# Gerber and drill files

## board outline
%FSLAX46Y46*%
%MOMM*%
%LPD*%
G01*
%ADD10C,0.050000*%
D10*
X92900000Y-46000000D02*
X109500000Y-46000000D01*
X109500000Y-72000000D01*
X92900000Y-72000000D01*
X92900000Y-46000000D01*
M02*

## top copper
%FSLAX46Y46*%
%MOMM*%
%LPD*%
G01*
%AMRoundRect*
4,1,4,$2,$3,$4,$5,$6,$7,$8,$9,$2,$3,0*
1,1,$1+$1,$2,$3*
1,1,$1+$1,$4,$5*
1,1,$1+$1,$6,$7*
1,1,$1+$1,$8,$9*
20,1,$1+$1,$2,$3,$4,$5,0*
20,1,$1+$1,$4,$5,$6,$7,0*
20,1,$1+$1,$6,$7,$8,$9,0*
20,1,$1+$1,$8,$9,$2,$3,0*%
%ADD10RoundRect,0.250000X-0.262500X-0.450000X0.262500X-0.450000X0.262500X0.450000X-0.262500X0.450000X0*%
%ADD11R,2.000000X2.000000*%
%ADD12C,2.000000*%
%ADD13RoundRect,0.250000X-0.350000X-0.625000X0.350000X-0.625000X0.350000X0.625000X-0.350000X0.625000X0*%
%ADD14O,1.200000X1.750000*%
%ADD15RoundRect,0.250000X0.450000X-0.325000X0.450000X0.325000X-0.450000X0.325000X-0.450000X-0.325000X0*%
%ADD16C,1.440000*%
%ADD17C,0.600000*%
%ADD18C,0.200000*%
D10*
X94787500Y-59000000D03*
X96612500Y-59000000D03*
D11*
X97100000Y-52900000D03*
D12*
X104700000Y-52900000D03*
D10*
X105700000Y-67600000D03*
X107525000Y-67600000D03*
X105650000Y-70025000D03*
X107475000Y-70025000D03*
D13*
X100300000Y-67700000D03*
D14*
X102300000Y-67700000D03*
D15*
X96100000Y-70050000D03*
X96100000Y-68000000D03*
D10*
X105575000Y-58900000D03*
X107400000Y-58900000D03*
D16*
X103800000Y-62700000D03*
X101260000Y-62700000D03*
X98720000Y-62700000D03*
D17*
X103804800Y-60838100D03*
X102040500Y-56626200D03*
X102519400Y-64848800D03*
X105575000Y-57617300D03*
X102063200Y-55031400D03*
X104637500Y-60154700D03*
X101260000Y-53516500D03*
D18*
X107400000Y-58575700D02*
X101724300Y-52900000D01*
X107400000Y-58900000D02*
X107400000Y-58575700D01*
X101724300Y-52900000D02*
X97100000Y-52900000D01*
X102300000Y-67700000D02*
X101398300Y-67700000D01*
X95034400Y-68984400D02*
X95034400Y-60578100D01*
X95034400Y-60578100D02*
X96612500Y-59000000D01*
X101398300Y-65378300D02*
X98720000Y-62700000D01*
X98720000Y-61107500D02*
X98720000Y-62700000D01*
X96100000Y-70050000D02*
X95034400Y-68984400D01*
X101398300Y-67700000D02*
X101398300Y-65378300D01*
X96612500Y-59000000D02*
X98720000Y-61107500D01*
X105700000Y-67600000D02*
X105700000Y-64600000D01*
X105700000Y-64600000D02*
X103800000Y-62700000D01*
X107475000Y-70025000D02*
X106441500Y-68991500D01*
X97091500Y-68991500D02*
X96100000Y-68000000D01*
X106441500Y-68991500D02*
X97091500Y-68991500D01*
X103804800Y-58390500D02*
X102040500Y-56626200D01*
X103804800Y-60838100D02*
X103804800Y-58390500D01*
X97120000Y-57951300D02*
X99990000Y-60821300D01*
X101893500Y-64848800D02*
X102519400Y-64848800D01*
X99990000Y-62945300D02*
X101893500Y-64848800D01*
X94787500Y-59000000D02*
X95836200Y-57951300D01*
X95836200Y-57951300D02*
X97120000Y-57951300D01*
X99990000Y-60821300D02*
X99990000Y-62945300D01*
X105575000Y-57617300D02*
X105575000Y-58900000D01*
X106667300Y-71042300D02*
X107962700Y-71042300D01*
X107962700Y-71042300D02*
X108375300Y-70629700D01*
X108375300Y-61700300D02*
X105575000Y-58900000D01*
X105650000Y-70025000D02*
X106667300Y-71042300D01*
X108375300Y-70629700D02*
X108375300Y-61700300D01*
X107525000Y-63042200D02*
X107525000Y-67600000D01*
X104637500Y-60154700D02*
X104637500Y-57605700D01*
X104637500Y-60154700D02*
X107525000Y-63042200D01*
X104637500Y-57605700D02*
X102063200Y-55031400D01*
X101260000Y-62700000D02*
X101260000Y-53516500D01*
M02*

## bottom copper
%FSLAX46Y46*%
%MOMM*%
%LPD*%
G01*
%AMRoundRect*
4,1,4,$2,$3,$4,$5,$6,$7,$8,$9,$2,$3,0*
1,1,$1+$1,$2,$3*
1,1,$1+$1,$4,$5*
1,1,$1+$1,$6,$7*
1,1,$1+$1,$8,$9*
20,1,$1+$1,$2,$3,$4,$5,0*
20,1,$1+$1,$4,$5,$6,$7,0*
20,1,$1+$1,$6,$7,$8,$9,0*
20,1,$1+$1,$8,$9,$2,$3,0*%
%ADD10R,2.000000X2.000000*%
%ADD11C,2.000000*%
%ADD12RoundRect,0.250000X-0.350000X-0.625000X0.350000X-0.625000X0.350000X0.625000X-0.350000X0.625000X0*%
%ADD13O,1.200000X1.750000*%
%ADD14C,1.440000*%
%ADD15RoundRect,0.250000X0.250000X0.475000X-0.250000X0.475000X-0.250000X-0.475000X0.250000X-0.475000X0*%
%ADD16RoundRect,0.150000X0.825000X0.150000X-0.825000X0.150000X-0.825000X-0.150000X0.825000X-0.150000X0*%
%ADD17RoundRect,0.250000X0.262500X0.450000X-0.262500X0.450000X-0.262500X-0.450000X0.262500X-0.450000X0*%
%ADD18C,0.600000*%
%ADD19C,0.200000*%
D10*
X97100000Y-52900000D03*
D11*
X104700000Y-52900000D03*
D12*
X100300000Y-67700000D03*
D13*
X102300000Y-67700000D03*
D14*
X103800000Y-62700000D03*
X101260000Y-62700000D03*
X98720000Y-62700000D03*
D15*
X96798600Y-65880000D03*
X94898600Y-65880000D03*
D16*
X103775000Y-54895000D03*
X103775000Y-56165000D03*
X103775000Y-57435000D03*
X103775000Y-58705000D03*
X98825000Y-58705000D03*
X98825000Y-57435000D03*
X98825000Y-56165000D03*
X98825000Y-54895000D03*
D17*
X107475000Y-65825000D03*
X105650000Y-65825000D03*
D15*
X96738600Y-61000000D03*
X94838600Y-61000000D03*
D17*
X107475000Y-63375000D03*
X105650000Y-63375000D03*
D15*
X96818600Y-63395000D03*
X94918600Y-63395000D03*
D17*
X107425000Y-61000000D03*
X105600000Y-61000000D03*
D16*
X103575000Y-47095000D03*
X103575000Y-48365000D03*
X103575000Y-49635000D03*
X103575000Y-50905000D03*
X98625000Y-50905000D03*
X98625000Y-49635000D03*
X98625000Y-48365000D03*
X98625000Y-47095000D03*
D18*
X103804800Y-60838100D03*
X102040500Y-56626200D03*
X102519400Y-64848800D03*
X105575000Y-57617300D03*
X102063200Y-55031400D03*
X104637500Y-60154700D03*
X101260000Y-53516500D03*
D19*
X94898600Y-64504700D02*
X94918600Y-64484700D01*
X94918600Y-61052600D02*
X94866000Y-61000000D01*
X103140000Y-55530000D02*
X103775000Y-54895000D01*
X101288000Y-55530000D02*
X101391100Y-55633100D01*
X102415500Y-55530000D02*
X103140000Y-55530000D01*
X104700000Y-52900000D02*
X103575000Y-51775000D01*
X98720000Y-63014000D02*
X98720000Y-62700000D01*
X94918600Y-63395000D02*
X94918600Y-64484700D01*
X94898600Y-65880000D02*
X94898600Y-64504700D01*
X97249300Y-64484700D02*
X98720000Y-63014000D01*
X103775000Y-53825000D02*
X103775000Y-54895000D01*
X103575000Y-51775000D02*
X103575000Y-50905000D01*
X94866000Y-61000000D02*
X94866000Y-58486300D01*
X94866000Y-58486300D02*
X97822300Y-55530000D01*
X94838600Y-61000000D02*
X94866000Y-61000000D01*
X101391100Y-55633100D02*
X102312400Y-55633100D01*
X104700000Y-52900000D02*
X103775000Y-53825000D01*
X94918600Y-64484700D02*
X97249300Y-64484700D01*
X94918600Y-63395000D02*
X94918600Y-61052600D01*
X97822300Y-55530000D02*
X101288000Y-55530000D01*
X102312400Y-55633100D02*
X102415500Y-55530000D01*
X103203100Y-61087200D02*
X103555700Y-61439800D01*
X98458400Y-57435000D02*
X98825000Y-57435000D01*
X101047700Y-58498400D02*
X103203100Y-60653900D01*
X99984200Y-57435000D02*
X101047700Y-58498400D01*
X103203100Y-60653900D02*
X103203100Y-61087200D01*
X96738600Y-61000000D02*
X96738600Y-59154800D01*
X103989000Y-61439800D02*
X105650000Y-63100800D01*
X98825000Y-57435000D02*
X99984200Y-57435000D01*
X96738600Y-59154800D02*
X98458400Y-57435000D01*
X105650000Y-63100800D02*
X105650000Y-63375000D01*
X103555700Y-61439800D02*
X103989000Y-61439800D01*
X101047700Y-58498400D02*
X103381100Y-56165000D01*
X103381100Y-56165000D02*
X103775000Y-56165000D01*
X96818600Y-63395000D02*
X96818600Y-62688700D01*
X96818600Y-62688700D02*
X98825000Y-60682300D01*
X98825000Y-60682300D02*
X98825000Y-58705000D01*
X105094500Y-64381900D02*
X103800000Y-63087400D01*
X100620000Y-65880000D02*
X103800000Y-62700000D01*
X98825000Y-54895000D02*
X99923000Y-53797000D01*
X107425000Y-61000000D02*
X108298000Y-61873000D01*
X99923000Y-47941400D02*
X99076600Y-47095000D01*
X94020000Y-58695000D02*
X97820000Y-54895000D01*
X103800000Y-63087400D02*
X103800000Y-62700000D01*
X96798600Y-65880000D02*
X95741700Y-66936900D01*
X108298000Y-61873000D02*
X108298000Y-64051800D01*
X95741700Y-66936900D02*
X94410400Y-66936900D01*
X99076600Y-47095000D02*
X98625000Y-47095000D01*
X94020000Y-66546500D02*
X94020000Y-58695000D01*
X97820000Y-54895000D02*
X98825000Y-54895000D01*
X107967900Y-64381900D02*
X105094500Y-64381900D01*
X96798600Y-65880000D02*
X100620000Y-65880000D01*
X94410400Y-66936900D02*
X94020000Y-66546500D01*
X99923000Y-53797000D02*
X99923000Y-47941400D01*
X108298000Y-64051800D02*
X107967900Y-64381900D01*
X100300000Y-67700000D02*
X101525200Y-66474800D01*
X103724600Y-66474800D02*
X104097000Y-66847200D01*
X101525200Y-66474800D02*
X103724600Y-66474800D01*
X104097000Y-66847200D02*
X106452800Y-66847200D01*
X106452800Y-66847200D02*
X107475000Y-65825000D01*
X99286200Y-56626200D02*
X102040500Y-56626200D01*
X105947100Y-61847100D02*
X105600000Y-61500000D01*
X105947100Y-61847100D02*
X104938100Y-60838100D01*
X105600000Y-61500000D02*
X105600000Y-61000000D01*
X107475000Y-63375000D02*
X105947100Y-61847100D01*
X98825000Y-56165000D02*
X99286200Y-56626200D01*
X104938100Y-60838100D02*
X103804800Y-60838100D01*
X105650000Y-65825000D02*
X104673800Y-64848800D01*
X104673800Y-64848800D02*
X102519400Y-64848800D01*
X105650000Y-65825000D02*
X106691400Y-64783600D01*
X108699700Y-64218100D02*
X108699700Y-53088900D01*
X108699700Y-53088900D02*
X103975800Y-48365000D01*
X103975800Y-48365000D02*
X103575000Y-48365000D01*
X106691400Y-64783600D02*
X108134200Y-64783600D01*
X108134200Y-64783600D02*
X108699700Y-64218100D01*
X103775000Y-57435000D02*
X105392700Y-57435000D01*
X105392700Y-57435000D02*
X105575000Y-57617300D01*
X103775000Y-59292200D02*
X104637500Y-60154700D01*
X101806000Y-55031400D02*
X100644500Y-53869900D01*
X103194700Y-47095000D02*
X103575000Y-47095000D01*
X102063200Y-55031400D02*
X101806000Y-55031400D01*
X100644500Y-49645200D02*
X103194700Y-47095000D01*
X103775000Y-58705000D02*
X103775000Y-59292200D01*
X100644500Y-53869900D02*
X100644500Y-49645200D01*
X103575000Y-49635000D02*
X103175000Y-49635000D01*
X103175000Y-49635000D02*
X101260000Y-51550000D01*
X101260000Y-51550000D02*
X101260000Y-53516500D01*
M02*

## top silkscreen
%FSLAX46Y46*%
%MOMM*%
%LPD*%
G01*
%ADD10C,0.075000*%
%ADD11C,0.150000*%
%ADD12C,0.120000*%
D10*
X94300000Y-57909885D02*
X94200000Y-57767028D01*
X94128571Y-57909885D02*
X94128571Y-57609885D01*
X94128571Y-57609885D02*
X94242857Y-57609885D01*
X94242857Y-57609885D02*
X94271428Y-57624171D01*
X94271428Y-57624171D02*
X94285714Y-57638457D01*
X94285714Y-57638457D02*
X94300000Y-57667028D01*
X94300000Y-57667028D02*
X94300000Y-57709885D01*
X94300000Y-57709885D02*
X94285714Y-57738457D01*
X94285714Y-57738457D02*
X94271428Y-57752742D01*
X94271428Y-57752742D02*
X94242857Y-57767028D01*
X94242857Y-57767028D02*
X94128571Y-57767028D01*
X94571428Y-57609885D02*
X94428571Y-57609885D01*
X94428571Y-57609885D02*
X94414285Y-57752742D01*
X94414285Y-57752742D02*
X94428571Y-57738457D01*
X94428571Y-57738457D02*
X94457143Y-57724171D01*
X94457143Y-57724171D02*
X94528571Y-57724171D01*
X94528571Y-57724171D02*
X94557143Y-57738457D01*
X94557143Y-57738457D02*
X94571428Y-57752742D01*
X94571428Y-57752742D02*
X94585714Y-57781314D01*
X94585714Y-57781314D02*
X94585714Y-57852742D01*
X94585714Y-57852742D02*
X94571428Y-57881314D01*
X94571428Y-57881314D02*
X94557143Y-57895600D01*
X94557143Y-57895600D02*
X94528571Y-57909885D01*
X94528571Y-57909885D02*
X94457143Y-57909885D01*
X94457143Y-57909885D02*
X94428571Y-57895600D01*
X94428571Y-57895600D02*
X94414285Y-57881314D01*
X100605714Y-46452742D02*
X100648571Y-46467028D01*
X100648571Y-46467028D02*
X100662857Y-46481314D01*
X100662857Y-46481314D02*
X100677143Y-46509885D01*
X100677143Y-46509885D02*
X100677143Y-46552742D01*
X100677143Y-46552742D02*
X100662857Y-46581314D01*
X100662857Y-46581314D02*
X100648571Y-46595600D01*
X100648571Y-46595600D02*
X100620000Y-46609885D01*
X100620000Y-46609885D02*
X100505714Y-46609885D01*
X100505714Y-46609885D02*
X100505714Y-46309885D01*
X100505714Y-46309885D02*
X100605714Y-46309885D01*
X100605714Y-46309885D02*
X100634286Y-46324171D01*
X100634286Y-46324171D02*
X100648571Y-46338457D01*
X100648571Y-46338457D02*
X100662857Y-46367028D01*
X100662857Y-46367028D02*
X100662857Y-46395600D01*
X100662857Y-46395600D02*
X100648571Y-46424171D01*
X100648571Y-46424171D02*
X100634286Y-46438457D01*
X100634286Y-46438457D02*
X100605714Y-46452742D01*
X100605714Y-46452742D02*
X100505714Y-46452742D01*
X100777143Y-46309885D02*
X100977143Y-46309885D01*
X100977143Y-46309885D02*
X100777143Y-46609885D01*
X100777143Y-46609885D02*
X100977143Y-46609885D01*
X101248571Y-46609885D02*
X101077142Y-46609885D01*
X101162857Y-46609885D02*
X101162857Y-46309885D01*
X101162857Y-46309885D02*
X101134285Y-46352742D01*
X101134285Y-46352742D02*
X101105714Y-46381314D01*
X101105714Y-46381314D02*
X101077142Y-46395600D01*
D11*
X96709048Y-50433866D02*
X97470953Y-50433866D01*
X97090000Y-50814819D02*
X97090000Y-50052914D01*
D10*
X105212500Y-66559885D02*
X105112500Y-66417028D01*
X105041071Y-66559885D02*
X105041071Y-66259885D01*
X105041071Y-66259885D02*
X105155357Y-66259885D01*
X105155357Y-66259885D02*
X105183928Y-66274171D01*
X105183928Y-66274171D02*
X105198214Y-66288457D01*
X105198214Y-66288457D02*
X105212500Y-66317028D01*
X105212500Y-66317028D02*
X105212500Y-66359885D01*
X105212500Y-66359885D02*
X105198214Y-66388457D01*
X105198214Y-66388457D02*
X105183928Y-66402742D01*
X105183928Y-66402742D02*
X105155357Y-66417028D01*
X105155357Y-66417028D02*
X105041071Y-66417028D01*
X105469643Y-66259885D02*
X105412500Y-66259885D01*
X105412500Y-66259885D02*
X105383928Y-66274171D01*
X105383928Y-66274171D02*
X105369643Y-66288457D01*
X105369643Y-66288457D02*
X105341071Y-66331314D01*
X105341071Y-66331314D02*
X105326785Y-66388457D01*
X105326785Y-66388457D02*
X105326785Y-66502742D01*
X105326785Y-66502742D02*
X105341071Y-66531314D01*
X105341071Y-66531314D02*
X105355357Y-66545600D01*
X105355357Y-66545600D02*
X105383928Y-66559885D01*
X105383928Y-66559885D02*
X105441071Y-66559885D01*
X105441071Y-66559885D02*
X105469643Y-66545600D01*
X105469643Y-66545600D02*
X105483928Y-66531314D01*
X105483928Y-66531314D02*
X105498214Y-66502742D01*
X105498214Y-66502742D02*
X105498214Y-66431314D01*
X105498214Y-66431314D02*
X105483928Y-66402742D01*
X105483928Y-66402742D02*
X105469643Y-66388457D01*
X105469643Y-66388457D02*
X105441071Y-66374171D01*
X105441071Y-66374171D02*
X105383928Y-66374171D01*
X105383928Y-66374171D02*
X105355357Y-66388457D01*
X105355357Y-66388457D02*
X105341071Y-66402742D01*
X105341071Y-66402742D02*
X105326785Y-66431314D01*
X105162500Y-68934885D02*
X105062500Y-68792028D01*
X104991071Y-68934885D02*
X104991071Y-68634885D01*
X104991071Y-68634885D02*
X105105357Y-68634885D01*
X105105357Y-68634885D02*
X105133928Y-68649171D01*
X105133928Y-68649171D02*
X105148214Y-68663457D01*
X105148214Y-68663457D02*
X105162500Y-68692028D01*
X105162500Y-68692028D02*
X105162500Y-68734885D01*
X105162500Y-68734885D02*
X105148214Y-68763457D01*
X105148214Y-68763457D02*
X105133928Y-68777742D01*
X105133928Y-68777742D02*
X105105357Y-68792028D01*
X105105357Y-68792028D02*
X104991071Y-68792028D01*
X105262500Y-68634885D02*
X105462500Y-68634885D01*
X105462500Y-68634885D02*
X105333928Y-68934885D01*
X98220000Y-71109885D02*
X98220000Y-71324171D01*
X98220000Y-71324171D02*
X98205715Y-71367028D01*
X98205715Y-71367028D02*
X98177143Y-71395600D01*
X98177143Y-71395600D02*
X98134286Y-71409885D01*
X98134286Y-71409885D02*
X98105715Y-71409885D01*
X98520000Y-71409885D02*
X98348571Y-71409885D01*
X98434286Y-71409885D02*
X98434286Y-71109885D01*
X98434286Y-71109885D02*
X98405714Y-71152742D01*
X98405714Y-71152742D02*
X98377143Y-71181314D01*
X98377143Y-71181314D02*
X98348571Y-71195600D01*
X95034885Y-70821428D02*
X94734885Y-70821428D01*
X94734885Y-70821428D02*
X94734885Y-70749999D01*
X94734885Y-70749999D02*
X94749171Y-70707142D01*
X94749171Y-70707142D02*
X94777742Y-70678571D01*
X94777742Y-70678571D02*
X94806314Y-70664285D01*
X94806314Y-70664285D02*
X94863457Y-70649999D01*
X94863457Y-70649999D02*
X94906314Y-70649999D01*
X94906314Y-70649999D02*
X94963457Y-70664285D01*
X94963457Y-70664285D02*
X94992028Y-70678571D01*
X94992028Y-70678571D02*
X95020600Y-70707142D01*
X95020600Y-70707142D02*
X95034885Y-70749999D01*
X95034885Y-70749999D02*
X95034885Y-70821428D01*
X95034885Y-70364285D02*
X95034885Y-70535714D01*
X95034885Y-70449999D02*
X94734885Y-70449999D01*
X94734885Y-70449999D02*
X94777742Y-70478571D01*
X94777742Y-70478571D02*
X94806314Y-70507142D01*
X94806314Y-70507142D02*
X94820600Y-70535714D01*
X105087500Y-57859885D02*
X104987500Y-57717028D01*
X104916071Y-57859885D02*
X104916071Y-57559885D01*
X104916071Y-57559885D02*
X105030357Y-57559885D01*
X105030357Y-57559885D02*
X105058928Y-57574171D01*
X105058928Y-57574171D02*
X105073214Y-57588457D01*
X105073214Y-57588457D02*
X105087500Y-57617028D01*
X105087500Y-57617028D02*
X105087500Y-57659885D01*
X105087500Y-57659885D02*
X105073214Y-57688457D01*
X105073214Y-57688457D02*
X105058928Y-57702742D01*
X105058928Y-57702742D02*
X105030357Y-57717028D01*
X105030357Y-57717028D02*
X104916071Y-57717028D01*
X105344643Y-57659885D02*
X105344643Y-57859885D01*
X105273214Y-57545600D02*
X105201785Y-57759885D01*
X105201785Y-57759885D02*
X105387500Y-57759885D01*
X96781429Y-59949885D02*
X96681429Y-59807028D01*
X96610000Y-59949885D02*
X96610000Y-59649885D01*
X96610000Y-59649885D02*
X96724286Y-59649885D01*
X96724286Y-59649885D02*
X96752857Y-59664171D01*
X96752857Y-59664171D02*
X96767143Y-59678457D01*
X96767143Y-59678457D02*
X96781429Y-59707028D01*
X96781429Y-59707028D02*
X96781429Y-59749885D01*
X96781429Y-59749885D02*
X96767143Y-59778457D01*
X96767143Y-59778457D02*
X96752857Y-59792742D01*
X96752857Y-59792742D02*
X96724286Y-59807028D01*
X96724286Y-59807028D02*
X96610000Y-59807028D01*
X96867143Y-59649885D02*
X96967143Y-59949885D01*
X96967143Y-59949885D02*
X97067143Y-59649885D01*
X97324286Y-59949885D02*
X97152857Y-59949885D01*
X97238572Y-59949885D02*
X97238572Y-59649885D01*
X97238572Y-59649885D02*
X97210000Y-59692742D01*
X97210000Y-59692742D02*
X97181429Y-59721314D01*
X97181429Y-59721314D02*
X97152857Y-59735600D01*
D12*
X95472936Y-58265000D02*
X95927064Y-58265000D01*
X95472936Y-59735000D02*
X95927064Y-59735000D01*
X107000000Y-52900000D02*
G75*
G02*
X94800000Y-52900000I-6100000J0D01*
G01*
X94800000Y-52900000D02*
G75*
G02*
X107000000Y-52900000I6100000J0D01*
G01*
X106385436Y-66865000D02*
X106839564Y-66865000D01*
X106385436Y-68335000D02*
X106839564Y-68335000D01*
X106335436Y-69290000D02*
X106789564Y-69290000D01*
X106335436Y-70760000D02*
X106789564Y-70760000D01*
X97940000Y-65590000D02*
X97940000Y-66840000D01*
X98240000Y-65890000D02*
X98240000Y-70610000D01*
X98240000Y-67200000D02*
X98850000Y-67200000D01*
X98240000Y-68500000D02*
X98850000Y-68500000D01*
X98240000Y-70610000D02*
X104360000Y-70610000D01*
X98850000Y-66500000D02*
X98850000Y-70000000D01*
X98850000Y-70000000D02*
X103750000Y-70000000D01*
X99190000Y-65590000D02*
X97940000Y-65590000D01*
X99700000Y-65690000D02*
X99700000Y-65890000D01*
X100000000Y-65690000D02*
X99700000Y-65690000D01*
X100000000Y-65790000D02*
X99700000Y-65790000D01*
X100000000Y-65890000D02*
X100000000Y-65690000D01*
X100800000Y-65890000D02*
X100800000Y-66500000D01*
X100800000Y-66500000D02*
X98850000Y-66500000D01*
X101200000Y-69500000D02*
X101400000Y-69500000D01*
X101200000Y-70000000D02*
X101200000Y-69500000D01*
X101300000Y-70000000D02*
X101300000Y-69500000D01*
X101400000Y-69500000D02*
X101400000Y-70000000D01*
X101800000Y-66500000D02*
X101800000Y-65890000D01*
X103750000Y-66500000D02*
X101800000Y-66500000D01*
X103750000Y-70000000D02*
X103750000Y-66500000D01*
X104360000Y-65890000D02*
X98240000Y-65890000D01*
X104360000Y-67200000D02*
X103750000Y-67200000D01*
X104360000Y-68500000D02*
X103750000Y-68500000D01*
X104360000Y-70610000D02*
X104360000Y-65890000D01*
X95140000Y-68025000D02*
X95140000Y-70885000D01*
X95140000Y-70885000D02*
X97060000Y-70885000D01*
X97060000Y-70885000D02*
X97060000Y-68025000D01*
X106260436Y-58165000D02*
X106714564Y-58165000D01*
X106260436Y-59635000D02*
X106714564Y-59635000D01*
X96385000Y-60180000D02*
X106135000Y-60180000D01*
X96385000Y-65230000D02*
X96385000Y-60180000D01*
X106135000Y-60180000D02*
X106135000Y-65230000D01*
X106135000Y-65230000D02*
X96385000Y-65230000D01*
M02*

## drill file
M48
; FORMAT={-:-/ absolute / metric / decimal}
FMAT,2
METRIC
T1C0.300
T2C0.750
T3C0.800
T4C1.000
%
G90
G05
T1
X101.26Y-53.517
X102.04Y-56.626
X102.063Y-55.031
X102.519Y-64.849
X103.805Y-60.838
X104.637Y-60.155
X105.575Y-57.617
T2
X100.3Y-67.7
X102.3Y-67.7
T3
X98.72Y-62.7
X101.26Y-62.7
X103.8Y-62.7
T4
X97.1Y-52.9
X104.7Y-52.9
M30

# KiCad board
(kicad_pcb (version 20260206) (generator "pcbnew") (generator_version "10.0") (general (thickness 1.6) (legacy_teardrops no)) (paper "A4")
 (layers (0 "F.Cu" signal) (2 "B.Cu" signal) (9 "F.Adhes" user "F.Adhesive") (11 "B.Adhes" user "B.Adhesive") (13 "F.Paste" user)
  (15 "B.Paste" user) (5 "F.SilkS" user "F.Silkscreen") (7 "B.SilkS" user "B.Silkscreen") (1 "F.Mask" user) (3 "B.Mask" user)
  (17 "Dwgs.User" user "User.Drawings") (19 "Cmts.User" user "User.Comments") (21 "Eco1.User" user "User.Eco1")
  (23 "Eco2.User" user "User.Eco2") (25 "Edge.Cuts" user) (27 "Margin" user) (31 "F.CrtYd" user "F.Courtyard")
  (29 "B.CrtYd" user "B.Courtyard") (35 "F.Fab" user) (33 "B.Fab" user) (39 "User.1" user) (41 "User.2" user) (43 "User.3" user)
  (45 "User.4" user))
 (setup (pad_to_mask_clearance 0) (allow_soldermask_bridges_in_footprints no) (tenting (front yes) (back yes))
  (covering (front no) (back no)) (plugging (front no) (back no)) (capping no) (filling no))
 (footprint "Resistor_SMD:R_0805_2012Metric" (layer "F.Cu") (at 95.7 59)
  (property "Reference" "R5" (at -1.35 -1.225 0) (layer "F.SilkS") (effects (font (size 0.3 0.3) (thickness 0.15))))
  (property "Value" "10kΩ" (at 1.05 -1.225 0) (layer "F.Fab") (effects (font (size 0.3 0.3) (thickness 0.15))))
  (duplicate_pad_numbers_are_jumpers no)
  (fp_line (start -0.227064 -0.735) (end 0.227064 -0.735) (stroke (width 0.12) (type solid)) (layer "F.SilkS"))
  (fp_line (start -0.227064 0.735) (end 0.227064 0.735) (stroke (width 0.12) (type solid)) (layer "F.SilkS"))
  (pad "1" smd roundrect (at -0.9125 0) (size 1.025 1.4) (layers "F.Cu" "F.Mask" "F.Paste") (roundrect_rratio 0.243902)
   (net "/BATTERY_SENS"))
  (pad "2" smd roundrect (at 0.9125 0) (size 1.025 1.4) (layers "F.Cu" "F.Mask" "F.Paste") (roundrect_rratio 0.243902) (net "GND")))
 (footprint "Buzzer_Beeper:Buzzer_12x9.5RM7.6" (layer "F.Cu") (at 97.1 52.9)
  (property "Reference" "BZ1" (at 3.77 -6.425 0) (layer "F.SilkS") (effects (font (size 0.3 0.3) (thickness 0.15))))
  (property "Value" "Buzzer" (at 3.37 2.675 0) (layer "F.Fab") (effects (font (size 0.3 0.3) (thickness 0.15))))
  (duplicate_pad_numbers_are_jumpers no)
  (fp_circle (center 3.8 0) (end 9.9 0) (stroke (width 0.12) (type solid)) (fill no) (layer "F.SilkS"))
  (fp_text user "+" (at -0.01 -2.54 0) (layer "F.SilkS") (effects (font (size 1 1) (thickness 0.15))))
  (pad "1" thru_hole rect (at 0 0) (size 2 2) (drill 1) (layers "*.Cu" "*.Mask") (remove_unused_layers no) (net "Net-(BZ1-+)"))
  (pad "2" thru_hole circle (at 7.6 0) (size 2 2) (drill 1) (layers "*.Cu" "*.Mask") (remove_unused_layers no) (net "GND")))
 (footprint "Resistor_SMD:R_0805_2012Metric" (layer "F.Cu") (at 106.6125 67.6)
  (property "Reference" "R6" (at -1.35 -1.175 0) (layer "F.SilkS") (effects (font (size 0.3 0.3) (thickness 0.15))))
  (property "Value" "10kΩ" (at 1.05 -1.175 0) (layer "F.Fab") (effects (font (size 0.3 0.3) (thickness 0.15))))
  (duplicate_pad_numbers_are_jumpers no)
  (fp_line (start -0.227064 -0.735) (end 0.227064 -0.735) (stroke (width 0.12) (type solid)) (layer "F.SilkS"))
  (fp_line (start -0.227064 0.735) (end 0.227064 0.735) (stroke (width 0.12) (type solid)) (layer "F.SilkS"))
  (pad "1" smd roundrect (at -0.9125 0) (size 1.025 1.4) (layers "F.Cu" "F.Mask" "F.Paste") (roundrect_rratio 0.243902) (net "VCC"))
  (pad "2" smd roundrect (at 0.9125 0) (size 1.025 1.4) (layers "F.Cu" "F.Mask" "F.Paste") (roundrect_rratio 0.243902) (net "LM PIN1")))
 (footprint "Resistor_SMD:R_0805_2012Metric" (layer "F.Cu") (at 106.5625 70.025)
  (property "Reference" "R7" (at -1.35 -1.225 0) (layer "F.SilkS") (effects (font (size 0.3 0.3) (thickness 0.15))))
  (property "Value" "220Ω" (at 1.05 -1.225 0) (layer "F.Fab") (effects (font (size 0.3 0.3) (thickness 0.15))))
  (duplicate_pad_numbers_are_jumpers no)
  (fp_line (start -0.227064 -0.735) (end 0.227064 -0.735) (stroke (width 0.12) (type solid)) (layer "F.SilkS"))
  (fp_line (start -0.227064 0.735) (end 0.227064 0.735) (stroke (width 0.12) (type solid)) (layer "F.SilkS"))
  (pad "1" smd roundrect (at -0.9125 0) (size 1.025 1.4) (layers "F.Cu" "F.Mask" "F.Paste") (roundrect_rratio 0.243902) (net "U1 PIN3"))
  (pad "2" smd roundrect (at 0.9125 0) (size 1.025 1.4) (layers "F.Cu" "F.Mask" "F.Paste") (roundrect_rratio 0.243902) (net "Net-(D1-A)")))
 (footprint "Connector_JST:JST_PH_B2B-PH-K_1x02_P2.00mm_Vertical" (layer "F.Cu") (at 100.3 67.7)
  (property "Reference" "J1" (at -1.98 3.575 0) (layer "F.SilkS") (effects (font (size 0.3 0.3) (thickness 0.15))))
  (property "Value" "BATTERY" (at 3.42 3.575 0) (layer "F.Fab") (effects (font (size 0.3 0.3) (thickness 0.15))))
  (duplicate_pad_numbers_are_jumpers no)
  (fp_line (start -2.36 -2.11) (end -2.36 -0.86) (stroke (width 0.12) (type solid)) (layer "F.SilkS"))
  (fp_line (start -2.06 -1.81) (end -2.06 2.91) (stroke (width 0.12) (type solid)) (layer "F.SilkS"))
  (fp_line (start -2.06 -0.5) (end -1.45 -0.5) (stroke (width 0.12) (type solid)) (layer "F.SilkS"))
  (fp_line (start -2.06 0.8) (end -1.45 0.8) (stroke (width 0.12) (type solid)) (layer "F.SilkS"))
  (fp_line (start -2.06 2.91) (end 4.06 2.91) (stroke (width 0.12) (type solid)) (layer "F.SilkS"))
  (fp_line (start -1.45 -1.2) (end -1.45 2.3) (stroke (width 0.12) (type solid)) (layer "F.SilkS"))
  (fp_line (start -1.45 2.3) (end 3.45 2.3) (stroke (width 0.12) (type solid)) (layer "F.SilkS"))
  (fp_line (start -1.11 -2.11) (end -2.36 -2.11) (stroke (width 0.12) (type solid)) (layer "F.SilkS"))
  (fp_line (start -0.6 -2.01) (end -0.6 -1.81) (stroke (width 0.12) (type solid)) (layer "F.SilkS"))
  (fp_line (start -0.3 -2.01) (end -0.6 -2.01) (stroke (width 0.12) (type solid)) (layer "F.SilkS"))
  (fp_line (start -0.3 -1.91) (end -0.6 -1.91) (stroke (width 0.12) (type solid)) (layer "F.SilkS"))
  (fp_line (start -0.3 -1.81) (end -0.3 -2.01) (stroke (width 0.12) (type solid)) (layer "F.SilkS"))
  (fp_line (start 0.5 -1.81) (end 0.5 -1.2) (stroke (width 0.12) (type solid)) (layer "F.SilkS"))
  (fp_line (start 0.5 -1.2) (end -1.45 -1.2) (stroke (width 0.12) (type solid)) (layer "F.SilkS"))
  (fp_line (start 0.9 1.8) (end 1.1 1.8) (stroke (width 0.12) (type solid)) (layer "F.SilkS"))
  (fp_line (start 0.9 2.3) (end 0.9 1.8) (stroke (width 0.12) (type solid)) (layer "F.SilkS"))
  (fp_line (start 1 2.3) (end 1 1.8) (stroke (width 0.12) (type solid)) (layer "F.SilkS"))
  (fp_line (start 1.1 1.8) (end 1.1 2.3) (stroke (width 0.12) (type solid)) (layer "F.SilkS"))
  (fp_line (start 1.5 -1.2) (end 1.5 -1.81) (stroke (width 0.12) (type solid)) (layer "F.SilkS"))
  (fp_line (start 3.45 -1.2) (end 1.5 -1.2) (stroke (width 0.12) (type solid)) (layer "F.SilkS"))
  (fp_line (start 3.45 2.3) (end 3.45 -1.2) (stroke (width 0.12) (type solid)) (layer "F.SilkS"))
  (fp_line (start 4.06 -1.81) (end -2.06 -1.81) (stroke (width 0.12) (type solid)) (layer "F.SilkS"))
  (fp_line (start 4.06 -0.5) (end 3.45 -0.5) (stroke (width 0.12) (type solid)) (layer "F.SilkS"))
  (fp_line (start 4.06 0.8) (end 3.45 0.8) (stroke (width 0.12) (type solid)) (layer "F.SilkS"))
  (fp_line (start 4.06 2.91) (end 4.06 -1.81) (stroke (width 0.12) (type solid)) (layer "F.SilkS"))
  (pad "1" thru_hole roundrect (at 0 0) (size 1.2 1.75) (drill 0.75) (layers "*.Cu" "*.Mask") (remove_unused_layers no)
   (roundrect_rratio 0.208333) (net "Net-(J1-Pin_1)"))
  (pad "2" thru_hole oval (at 2 0) (size 1.2 1.75) (drill 0.75) (layers "*.Cu" "*.Mask") (remove_unused_layers no) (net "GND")))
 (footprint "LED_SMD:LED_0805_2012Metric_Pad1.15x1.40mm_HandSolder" (layer "F.Cu") (at 96.1 69.025 90)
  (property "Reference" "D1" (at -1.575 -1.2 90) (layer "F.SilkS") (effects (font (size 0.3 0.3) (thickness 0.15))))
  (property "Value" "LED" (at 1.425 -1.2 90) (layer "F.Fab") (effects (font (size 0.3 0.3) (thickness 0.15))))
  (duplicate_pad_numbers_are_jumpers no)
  (fp_line (start 1 -0.96) (end -1.86 -0.96) (stroke (width 0.12) (type solid)) (layer "F.SilkS"))
  (fp_line (start -1.86 -0.96) (end -1.86 0.96) (stroke (width 0.12) (type solid)) (layer "F.SilkS"))
  (fp_line (start -1.86 0.96) (end 1 0.96) (stroke (width 0.12) (type solid)) (layer "F.SilkS"))
  (pad "1" smd roundrect (at -1.025 0 90) (size 1.15 1.4) (layers "F.Cu" "F.Mask" "F.Paste") (roundrect_rratio 0.217391) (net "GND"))
  (pad "2" smd roundrect (at 1.025 0 90) (size 1.15 1.4) (layers "F.Cu" "F.Mask" "F.Paste") (roundrect_rratio 0.217391) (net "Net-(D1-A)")))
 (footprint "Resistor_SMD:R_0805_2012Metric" (layer "F.Cu") (at 106.4875 58.9)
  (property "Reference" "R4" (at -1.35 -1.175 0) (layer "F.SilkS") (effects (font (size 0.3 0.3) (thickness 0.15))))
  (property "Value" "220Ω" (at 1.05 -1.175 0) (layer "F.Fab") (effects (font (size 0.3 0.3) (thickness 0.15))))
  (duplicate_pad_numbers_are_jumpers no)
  (fp_line (start -0.227064 -0.735) (end 0.227064 -0.735) (stroke (width 0.12) (type solid)) (layer "F.SilkS"))
  (fp_line (start -0.227064 0.735) (end 0.227064 0.735) (stroke (width 0.12) (type solid)) (layer "F.SilkS"))
  (pad "1" smd roundrect (at -0.9125 0) (size 1.025 1.4) (layers "F.Cu" "F.Mask" "F.Paste") (roundrect_rratio 0.243902) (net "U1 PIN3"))
  (pad "2" smd roundrect (at 0.9125 0) (size 1.025 1.4) (layers "F.Cu" "F.Mask" "F.Paste") (roundrect_rratio 0.243902) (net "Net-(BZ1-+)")))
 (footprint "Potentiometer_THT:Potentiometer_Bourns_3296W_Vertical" (layer "F.Cu") (at 103.8 62.7)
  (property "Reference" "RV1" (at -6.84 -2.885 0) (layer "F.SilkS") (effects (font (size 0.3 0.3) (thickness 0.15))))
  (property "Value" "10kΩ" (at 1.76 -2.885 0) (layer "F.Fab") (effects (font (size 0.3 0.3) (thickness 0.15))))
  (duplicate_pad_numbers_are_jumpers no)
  (fp_line (start -7.415 -2.52) (end 2.335 -2.52) (stroke (width 0.12) (type solid)) (layer "F.SilkS"))
  (fp_line (start -7.415 2.53) (end -7.415 -2.52) (stroke (width 0.12) (type solid)) (layer "F.SilkS"))
  (fp_line (start 2.335 -2.52) (end 2.335 2.53) (stroke (width 0.12) (type solid)) (layer "F.SilkS"))
  (fp_line (start 2.335 2.53) (end -7.415 2.53) (stroke (width 0.12) (type solid)) (layer "F.SilkS"))
  (pad "1" thru_hole circle (at 0 0) (size 1.44 1.44) (drill 0.8) (layers "*.Cu" "*.Mask") (remove_unused_layers no) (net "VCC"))
  (pad "2" thru_hole circle (at -2.54 0) (size 1.44 1.44) (drill 0.8) (layers "*.Cu" "*.Mask") (remove_unused_layers no) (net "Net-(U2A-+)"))
  (pad "3" thru_hole circle (at -5.08 0) (size 1.44 1.44) (drill 0.8) (layers "*.Cu" "*.Mask") (remove_unused_layers no) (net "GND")))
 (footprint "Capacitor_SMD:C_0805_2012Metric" (layer "B.Cu") (at 95.8486 65.88 180)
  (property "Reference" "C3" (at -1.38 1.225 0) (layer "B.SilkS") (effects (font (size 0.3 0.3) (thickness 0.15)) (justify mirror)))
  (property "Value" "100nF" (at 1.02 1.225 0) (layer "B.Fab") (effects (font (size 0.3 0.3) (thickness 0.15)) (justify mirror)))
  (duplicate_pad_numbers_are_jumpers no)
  (pad "1" smd roundrect (at -0.95 0 180) (size 1 1.45) (layers "B.Cu" "B.Mask" "B.Paste") (roundrect_rratio 0.25) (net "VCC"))
  (pad "2" smd roundrect (at 0.95 0 180) (size 1 1.45) (layers "B.Cu" "B.Mask" "B.Paste") (roundrect_rratio 0.25) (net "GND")))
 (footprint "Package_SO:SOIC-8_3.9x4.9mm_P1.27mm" (layer "B.Cu") (at 101.3 56.8 180)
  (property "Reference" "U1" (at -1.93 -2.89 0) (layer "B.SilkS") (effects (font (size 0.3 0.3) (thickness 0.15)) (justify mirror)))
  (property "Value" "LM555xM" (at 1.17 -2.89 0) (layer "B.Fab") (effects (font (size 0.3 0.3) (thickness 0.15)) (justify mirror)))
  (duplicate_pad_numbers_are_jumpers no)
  (pad "1" smd roundrect (at -2.475 1.905 180) (size 1.95 0.6) (layers "B.Cu" "B.Mask" "B.Paste") (roundrect_rratio 0.25) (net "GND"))
  (pad "2" smd roundrect (at -2.475 0.635 180) (size 1.95 0.6) (layers "B.Cu" "B.Mask" "B.Paste") (roundrect_rratio 0.25) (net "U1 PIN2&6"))
  (pad "3" smd roundrect (at -2.475 -0.635 180) (size 1.95 0.6) (layers "B.Cu" "B.Mask" "B.Paste") (roundrect_rratio 0.25) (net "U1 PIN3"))
  (pad "4" smd roundrect (at -2.475 -1.905 180) (size 1.95 0.6) (layers "B.Cu" "B.Mask" "B.Paste") (roundrect_rratio 0.25) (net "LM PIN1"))
  (pad "5" smd roundrect (at 2.475 -1.905 180) (size 1.95 0.6) (layers "B.Cu" "B.Mask" "B.Paste") (roundrect_rratio 0.25) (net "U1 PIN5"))
  (pad "6" smd roundrect (at 2.475 -0.635 180) (size 1.95 0.6) (layers "B.Cu" "B.Mask" "B.Paste") (roundrect_rratio 0.25) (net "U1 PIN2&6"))
  (pad "7" smd roundrect (at 2.475 0.635 180) (size 1.95 0.6) (layers "B.Cu" "B.Mask" "B.Paste") (roundrect_rratio 0.25) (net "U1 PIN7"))
  (pad "8" smd roundrect (at 2.475 1.905 180) (size 1.95 0.6) (layers "B.Cu" "B.Mask" "B.Paste") (roundrect_rratio 0.25) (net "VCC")))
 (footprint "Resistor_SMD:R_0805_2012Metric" (layer "B.Cu") (at 106.5625 65.825 180)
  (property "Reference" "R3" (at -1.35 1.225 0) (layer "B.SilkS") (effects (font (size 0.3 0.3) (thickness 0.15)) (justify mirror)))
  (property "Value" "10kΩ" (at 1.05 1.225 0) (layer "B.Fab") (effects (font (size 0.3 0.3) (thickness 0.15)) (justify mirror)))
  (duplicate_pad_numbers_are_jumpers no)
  (pad "1" smd roundrect (at -0.9125 0 180) (size 1.025 1.4) (layers "B.Cu" "B.Mask" "B.Paste") (roundrect_rratio 0.243902)
   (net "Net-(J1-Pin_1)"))
  (pad "2" smd roundrect (at 0.9125 0 180) (size 1.025 1.4) (layers "B.Cu" "B.Mask" "B.Paste") (roundrect_rratio 0.243902)
   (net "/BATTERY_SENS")))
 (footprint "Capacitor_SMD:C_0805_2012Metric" (layer "B.Cu") (at 95.7886 61 180)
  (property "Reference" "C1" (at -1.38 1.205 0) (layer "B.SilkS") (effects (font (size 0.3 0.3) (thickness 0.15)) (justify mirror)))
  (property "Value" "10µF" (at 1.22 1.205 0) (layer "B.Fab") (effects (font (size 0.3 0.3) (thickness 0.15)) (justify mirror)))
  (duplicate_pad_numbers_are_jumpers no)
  (pad "1" smd roundrect (at -0.95 0 180) (size 1 1.45) (layers "B.Cu" "B.Mask" "B.Paste") (roundrect_rratio 0.25) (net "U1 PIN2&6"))
  (pad "2" smd roundrect (at 0.95 0 180) (size 1 1.45) (layers "B.Cu" "B.Mask" "B.Paste") (roundrect_rratio 0.25) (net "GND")))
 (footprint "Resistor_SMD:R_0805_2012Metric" (layer "B.Cu") (at 106.5625 63.375 180)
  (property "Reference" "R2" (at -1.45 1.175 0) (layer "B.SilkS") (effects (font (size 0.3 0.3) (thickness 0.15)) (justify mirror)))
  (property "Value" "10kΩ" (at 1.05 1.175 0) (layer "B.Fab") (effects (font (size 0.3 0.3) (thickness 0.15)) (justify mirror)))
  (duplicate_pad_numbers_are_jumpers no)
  (pad "1" smd roundrect (at -0.9125 0 180) (size 1.025 1.4) (layers "B.Cu" "B.Mask" "B.Paste") (roundrect_rratio 0.243902) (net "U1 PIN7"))
  (pad "2" smd roundrect (at 0.9125 0 180) (size 1.025 1.4) (layers "B.Cu" "B.Mask" "B.Paste") (roundrect_rratio 0.243902) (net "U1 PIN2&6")))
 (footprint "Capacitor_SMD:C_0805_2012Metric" (layer "B.Cu") (at 95.8686 63.395 180)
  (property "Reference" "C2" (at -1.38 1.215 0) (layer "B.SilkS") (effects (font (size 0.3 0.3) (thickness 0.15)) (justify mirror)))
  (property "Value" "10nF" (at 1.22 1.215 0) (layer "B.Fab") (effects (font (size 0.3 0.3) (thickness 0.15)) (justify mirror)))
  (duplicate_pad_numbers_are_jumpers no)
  (pad "1" smd roundrect (at -0.95 0 180) (size 1 1.45) (layers "B.Cu" "B.Mask" "B.Paste") (roundrect_rratio 0.25) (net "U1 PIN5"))
  (pad "2" smd roundrect (at 0.95 0 180) (size 1 1.45) (layers "B.Cu" "B.Mask" "B.Paste") (roundrect_rratio 0.25) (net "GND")))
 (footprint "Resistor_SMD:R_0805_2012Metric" (layer "B.Cu") (at 106.5125 61 180)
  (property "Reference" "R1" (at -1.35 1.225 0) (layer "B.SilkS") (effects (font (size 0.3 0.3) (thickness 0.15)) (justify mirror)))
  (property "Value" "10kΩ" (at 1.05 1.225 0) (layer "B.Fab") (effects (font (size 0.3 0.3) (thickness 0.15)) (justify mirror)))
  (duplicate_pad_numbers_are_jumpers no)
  (pad "1" smd roundrect (at -0.9125 0 180) (size 1.025 1.4) (layers "B.Cu" "B.Mask" "B.Paste") (roundrect_rratio 0.243902) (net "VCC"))
  (pad "2" smd roundrect (at 0.9125 0 180) (size 1.025 1.4) (layers "B.Cu" "B.Mask" "B.Paste") (roundrect_rratio 0.243902) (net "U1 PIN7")))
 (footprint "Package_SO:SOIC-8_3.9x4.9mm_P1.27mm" (layer "B.Cu") (at 101.1 49 180)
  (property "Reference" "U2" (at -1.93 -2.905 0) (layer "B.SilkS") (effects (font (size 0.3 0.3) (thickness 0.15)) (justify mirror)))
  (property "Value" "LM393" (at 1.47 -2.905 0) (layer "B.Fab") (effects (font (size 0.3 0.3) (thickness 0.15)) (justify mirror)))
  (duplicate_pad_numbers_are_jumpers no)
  (pad "1" smd roundrect (at -2.475 1.905 180) (size 1.95 0.6) (layers "B.Cu" "B.Mask" "B.Paste") (roundrect_rratio 0.25) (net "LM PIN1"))
  (pad "2" smd roundrect (at -2.475 0.635 180) (size 1.95 0.6) (layers "B.Cu" "B.Mask" "B.Paste") (roundrect_rratio 0.25)
   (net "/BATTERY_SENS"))
  (pad "3" smd roundrect (at -2.475 -0.635 180) (size 1.95 0.6) (layers "B.Cu" "B.Mask" "B.Paste") (roundrect_rratio 0.25)
   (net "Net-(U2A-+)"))
  (pad "4" smd roundrect (at -2.475 -1.905 180) (size 1.95 0.6) (layers "B.Cu" "B.Mask" "B.Paste") (roundrect_rratio 0.25) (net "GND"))
  (pad "5" smd roundrect (at 2.475 -1.905 180) (size 1.95 0.6) (layers "B.Cu" "B.Mask" "B.Paste") (roundrect_rratio 0.25)
   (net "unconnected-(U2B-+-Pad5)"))
  (pad "6" smd roundrect (at 2.475 -0.635 180) (size 1.95 0.6) (layers "B.Cu" "B.Mask" "B.Paste") (roundrect_rratio 0.25)
   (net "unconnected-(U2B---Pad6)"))
  (pad "7" smd roundrect (at 2.475 0.635 180) (size 1.95 0.6) (layers "B.Cu" "B.Mask" "B.Paste") (roundrect_rratio 0.25)
   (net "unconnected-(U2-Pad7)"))
  (pad "8" smd roundrect (at 2.475 1.905 180) (size 1.95 0.6) (layers "B.Cu" "B.Mask" "B.Paste") (roundrect_rratio 0.25) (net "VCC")))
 (gr_rect (start 92.9 46) (end 109.5 72) (stroke (width 0.05) (type default)) (fill no) (layer "Edge.Cuts"))
 (segment (start 107.4 58.5757) (end 101.7243 52.9) (width 0.2) (layer "F.Cu") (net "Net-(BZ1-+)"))
 (segment (start 107.4 58.9) (end 107.4 58.5757) (width 0.2) (layer "F.Cu") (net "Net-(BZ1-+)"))
 (segment (start 101.7243 52.9) (end 97.1 52.9) (width 0.2) (layer "F.Cu") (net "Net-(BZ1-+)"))
 (segment (start 102.3 67.7) (end 101.3983 67.7) (width 0.2) (layer "F.Cu") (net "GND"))
 (segment (start 95.0344 68.9844) (end 95.0344 60.5781) (width 0.2) (layer "F.Cu") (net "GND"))
 (segment (start 95.0344 60.5781) (end 96.6125 59) (width 0.2) (layer "F.Cu") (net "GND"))
 (segment (start 101.3983 65.3783) (end 98.72 62.7) (width 0.2) (layer "F.Cu") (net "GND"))
 (segment (start 98.72 61.1075) (end 98.72 62.7) (width 0.2) (layer "F.Cu") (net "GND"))
 (segment (start 96.1 70.05) (end 95.0344 68.9844) (width 0.2) (layer "F.Cu") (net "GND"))
 (segment (start 101.3983 67.7) (end 101.3983 65.3783) (width 0.2) (layer "F.Cu") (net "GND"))
 (segment (start 96.6125 59) (end 98.72 61.1075) (width 0.2) (layer "F.Cu") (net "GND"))
 (segment (start 94.8986 64.5047) (end 94.9186 64.4847) (width 0.2) (layer "B.Cu") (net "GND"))
 (segment (start 94.9186 61.0526) (end 94.866 61) (width 0.2) (layer "B.Cu") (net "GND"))
 (segment (start 103.14 55.53) (end 103.775 54.895) (width 0.2) (layer "B.Cu") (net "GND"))
 (segment (start 101.288 55.53) (end 101.3911 55.6331) (width 0.2) (layer "B.Cu") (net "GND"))
 (segment (start 102.4155 55.53) (end 103.14 55.53) (width 0.2) (layer "B.Cu") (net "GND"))
 (segment (start 104.7 52.9) (end 103.575 51.775) (width 0.2) (layer "B.Cu") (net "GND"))
 (segment (start 98.72 63.014) (end 98.72 62.7) (width 0.2) (layer "B.Cu") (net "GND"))
 (segment (start 94.9186 63.395) (end 94.9186 64.4847) (width 0.2) (layer "B.Cu") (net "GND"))
 (segment (start 94.8986 65.88) (end 94.8986 64.5047) (width 0.2) (layer "B.Cu") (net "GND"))
 (segment (start 97.2493 64.4847) (end 98.72 63.014) (width 0.2) (layer "B.Cu") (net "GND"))
 (segment (start 103.775 53.825) (end 103.775 54.895) (width 0.2) (layer "B.Cu") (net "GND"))
 (segment (start 103.575 51.775) (end 103.575 50.905) (width 0.2) (layer "B.Cu") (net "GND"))
 (segment (start 94.866 61) (end 94.866 58.4863) (width 0.2) (layer "B.Cu") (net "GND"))
 (segment (start 94.866 58.4863) (end 97.8223 55.53) (width 0.2) (layer "B.Cu") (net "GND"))
 (segment (start 94.8386 61) (end 94.866 61) (width 0.2) (layer "B.Cu") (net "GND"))
 (segment (start 101.3911 55.6331) (end 102.3124 55.6331) (width 0.2) (layer "B.Cu") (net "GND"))
 (segment (start 104.7 52.9) (end 103.775 53.825) (width 0.2) (layer "B.Cu") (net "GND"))
 (segment (start 94.9186 64.4847) (end 97.2493 64.4847) (width 0.2) (layer "B.Cu") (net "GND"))
 (segment (start 94.9186 63.395) (end 94.9186 61.0526) (width 0.2) (layer "B.Cu") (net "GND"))
 (segment (start 97.8223 55.53) (end 101.288 55.53) (width 0.2) (layer "B.Cu") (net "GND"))
 (segment (start 102.3124 55.6331) (end 102.4155 55.53) (width 0.2) (layer "B.Cu") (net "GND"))
 (segment (start 103.2031 61.0872) (end 103.5557 61.4398) (width 0.2) (layer "B.Cu") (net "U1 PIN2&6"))
 (segment (start 98.4584 57.435) (end 98.825 57.435) (width 0.2) (layer "B.Cu") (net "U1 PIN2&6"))
 (segment (start 101.0477 58.4984) (end 103.2031 60.6539) (width 0.2) (layer "B.Cu") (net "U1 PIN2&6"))
 (segment (start 99.9842 57.435) (end 101.0477 58.4984) (width 0.2) (layer "B.Cu") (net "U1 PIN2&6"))
 (segment (start 103.2031 60.6539) (end 103.2031 61.0872) (width 0.2) (layer "B.Cu") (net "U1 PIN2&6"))
 (segment (start 96.7386 61) (end 96.7386 59.1548) (width 0.2) (layer "B.Cu") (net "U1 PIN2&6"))
 (segment (start 103.989 61.4398) (end 105.65 63.1008) (width 0.2) (layer "B.Cu") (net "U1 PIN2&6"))
 (segment (start 98.825 57.435) (end 99.9842 57.435) (width 0.2) (layer "B.Cu") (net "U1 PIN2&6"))
 (segment (start 96.7386 59.1548) (end 98.4584 57.435) (width 0.2) (layer "B.Cu") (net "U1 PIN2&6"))
 (segment (start 105.65 63.1008) (end 105.65 63.375) (width 0.2) (layer "B.Cu") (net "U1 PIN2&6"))
 (segment (start 103.5557 61.4398) (end 103.989 61.4398) (width 0.2) (layer "B.Cu") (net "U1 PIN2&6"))
 (segment (start 101.0477 58.4984) (end 103.3811 56.165) (width 0.2) (layer "B.Cu") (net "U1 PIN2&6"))
 (segment (start 103.3811 56.165) (end 103.775 56.165) (width 0.2) (layer "B.Cu") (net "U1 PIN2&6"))
 (segment (start 96.8186 63.395) (end 96.8186 62.6887) (width 0.2) (layer "B.Cu") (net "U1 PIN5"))
 (segment (start 96.8186 62.6887) (end 98.825 60.6823) (width 0.2) (layer "B.Cu") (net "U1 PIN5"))
 (segment (start 98.825 60.6823) (end 98.825 58.705) (width 0.2) (layer "B.Cu") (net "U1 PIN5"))
 (segment (start 105.7 67.6) (end 105.7 64.6) (width 0.2) (layer "F.Cu") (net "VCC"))
 (segment (start 105.7 64.6) (end 103.8 62.7) (width 0.2) (layer "F.Cu") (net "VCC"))
 (segment (start 105.0945 64.3819) (end 103.8 63.0874) (width 0.2) (layer "B.Cu") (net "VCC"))
 (segment (start 100.62 65.88) (end 103.8 62.7) (width 0.2) (layer "B.Cu") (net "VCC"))
 (segment (start 98.825 54.895) (end 99.923 53.797) (width 0.2) (layer "B.Cu") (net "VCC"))
 (segment (start 107.425 61) (end 108.298 61.873) (width 0.2) (layer "B.Cu") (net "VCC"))
 (segment (start 99.923 47.9414) (end 99.0766 47.095) (width 0.2) (layer "B.Cu") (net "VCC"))
 (segment (start 94.02 58.695) (end 97.82 54.895) (width 0.2) (layer "B.Cu") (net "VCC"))
 (segment (start 103.8 63.0874) (end 103.8 62.7) (width 0.2) (layer "B.Cu") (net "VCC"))
 (segment (start 96.7986 65.88) (end 95.7417 66.9369) (width 0.2) (layer "B.Cu") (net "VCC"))
 (segment (start 108.298 61.873) (end 108.298 64.0518) (width 0.2) (layer "B.Cu") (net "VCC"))
 (segment (start 95.7417 66.9369) (end 94.4104 66.9369) (width 0.2) (layer "B.Cu") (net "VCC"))
 (segment (start 99.0766 47.095) (end 98.625 47.095) (width 0.2) (layer "B.Cu") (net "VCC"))
 (segment (start 94.02 66.5465) (end 94.02 58.695) (width 0.2) (layer "B.Cu") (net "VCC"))
 (segment (start 97.82 54.895) (end 98.825 54.895) (width 0.2) (layer "B.Cu") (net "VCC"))
 (segment (start 107.9679 64.3819) (end 105.0945 64.3819) (width 0.2) (layer "B.Cu") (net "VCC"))
 (segment (start 96.7986 65.88) (end 100.62 65.88) (width 0.2) (layer "B.Cu") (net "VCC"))
 (segment (start 94.4104 66.9369) (end 94.02 66.5465) (width 0.2) (layer "B.Cu") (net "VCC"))
 (segment (start 99.923 53.797) (end 99.923 47.9414) (width 0.2) (layer "B.Cu") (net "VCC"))
 (segment (start 108.298 64.0518) (end 107.9679 64.3819) (width 0.2) (layer "B.Cu") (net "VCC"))
 (segment (start 107.475 70.025) (end 106.4415 68.9915) (width 0.2) (layer "F.Cu") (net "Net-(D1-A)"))
 (segment (start 97.0915 68.9915) (end 96.1 68) (width 0.2) (layer "F.Cu") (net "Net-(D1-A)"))
 (segment (start 106.4415 68.9915) (end 97.0915 68.9915) (width 0.2) (layer "F.Cu") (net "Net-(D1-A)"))
 (segment (start 100.3 67.7) (end 101.5252 66.4748) (width 0.2) (layer "B.Cu") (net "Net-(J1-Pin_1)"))
 (segment (start 103.7246 66.4748) (end 104.097 66.8472) (width 0.2) (layer "B.Cu") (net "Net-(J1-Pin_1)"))
 (segment (start 101.5252 66.4748) (end 103.7246 66.4748) (width 0.2) (layer "B.Cu") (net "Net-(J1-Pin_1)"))
 (segment (start 104.097 66.8472) (end 106.4528 66.8472) (width 0.2) (layer "B.Cu") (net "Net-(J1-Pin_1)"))
 (segment (start 106.4528 66.8472) (end 107.475 65.825) (width 0.2) (layer "B.Cu") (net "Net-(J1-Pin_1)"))
 (segment (start 103.8048 58.3905) (end 102.0405 56.6262) (width 0.2) (layer "F.Cu") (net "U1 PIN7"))
 (segment (start 103.8048 60.8381) (end 103.8048 58.3905) (width 0.2) (layer "F.Cu") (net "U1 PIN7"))
 (via (at 103.8048 60.8381) (size 0.6) (drill 0.3) (layers "F.Cu" "B.Cu") (capping no) (covering (front no) (back no))
  (plugging (front no) (back no)) (filling no) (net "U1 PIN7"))
 (via (at 102.0405 56.6262) (size 0.6) (drill 0.3) (layers "F.Cu" "B.Cu") (capping no) (covering (front no) (back no))
  (plugging (front no) (back no)) (filling no) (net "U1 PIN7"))
 (segment (start 99.2862 56.6262) (end 102.0405 56.6262) (width 0.2) (layer "B.Cu") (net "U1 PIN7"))
 (segment (start 105.9471 61.8471) (end 105.6 61.5) (width 0.2) (layer "B.Cu") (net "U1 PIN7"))
 (segment (start 105.9471 61.8471) (end 104.9381 60.8381) (width 0.2) (layer "B.Cu") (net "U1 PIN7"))
 (segment (start 105.6 61.5) (end 105.6 61) (width 0.2) (layer "B.Cu") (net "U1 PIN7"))
 (segment (start 107.475 63.375) (end 105.9471 61.8471) (width 0.2) (layer "B.Cu") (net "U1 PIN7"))
 (segment (start 98.825 56.165) (end 99.2862 56.6262) (width 0.2) (layer "B.Cu") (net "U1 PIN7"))
 (segment (start 104.9381 60.8381) (end 103.8048 60.8381) (width 0.2) (layer "B.Cu") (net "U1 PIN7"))
 (segment (start 97.12 57.9513) (end 99.99 60.8213) (width 0.2) (layer "F.Cu") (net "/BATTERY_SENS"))
 (segment (start 101.8935 64.8488) (end 102.5194 64.8488) (width 0.2) (layer "F.Cu") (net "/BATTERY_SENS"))
 (segment (start 99.99 62.9453) (end 101.8935 64.8488) (width 0.2) (layer "F.Cu") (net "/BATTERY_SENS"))
 (segment (start 94.7875 59) (end 95.8362 57.9513) (width 0.2) (layer "F.Cu") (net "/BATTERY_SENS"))
 (segment (start 95.8362 57.9513) (end 97.12 57.9513) (width 0.2) (layer "F.Cu") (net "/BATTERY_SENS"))
 (segment (start 99.99 60.8213) (end 99.99 62.9453) (width 0.2) (layer "F.Cu") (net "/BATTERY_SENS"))
 (via (at 102.5194 64.8488) (size 0.6) (drill 0.3) (layers "F.Cu" "B.Cu") (capping no) (covering (front no) (back no))
  (plugging (front no) (back no)) (filling no) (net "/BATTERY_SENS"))
 (segment (start 105.65 65.825) (end 104.6738 64.8488) (width 0.2) (layer "B.Cu") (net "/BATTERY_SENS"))
 (segment (start 104.6738 64.8488) (end 102.5194 64.8488) (width 0.2) (layer "B.Cu") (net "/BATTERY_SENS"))
 (segment (start 105.65 65.825) (end 106.6914 64.7836) (width 0.2) (layer "B.Cu") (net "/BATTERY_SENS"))
 (segment (start 108.6997 64.2181) (end 108.6997 53.0889) (width 0.2) (layer "B.Cu") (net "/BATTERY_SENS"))
 (segment (start 108.6997 53.0889) (end 103.9758 48.365) (width 0.2) (layer "B.Cu") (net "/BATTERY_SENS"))
 (segment (start 103.9758 48.365) (end 103.575 48.365) (width 0.2) (layer "B.Cu") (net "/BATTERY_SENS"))
 (segment (start 106.6914 64.7836) (end 108.1342 64.7836) (width 0.2) (layer "B.Cu") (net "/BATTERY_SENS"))
 (segment (start 108.1342 64.7836) (end 108.6997 64.2181) (width 0.2) (layer "B.Cu") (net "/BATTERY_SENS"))
 (segment (start 105.575 57.6173) (end 105.575 58.9) (width 0.2) (layer "F.Cu") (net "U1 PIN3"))
 (segment (start 106.6673 71.0423) (end 107.9627 71.0423) (width 0.2) (layer "F.Cu") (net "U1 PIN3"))
 (segment (start 107.9627 71.0423) (end 108.3753 70.6297) (width 0.2) (layer "F.Cu") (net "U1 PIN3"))
 (segment (start 108.3753 61.7003) (end 105.575 58.9) (width 0.2) (layer "F.Cu") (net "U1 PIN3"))
 (segment (start 105.65 70.025) (end 106.6673 71.0423) (width 0.2) (layer "F.Cu") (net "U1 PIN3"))
 (segment (start 108.3753 70.6297) (end 108.3753 61.7003) (width 0.2) (layer "F.Cu") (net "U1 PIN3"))
 (via (at 105.575 57.6173) (size 0.6) (drill 0.3) (layers "F.Cu" "B.Cu") (capping no) (covering (front no) (back no))
  (plugging (front no) (back no)) (filling no) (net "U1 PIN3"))
 (segment (start 103.775 57.435) (end 105.3927 57.435) (width 0.2) (layer "B.Cu") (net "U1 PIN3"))
 (segment (start 105.3927 57.435) (end 105.575 57.6173) (width 0.2) (layer "B.Cu") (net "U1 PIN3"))
 (segment (start 107.525 63.0422) (end 107.525 67.6) (width 0.2) (layer "F.Cu") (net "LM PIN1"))
 (segment (start 104.6375 60.1547) (end 104.6375 57.6057) (width 0.2) (layer "F.Cu") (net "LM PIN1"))
 (segment (start 104.6375 60.1547) (end 107.525 63.0422) (width 0.2) (layer "F.Cu") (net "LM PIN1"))
 (segment (start 104.6375 57.6057) (end 102.0632 55.0314) (width 0.2) (layer "F.Cu") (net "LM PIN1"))
 (via (at 102.0632 55.0314) (size 0.6) (drill 0.3) (layers "F.Cu" "B.Cu") (capping no) (covering (front no) (back no))
  (plugging (front no) (back no)) (filling no) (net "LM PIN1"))
 (via (at 104.6375 60.1547) (size 0.6) (drill 0.3) (layers "F.Cu" "B.Cu") (capping no) (covering (front no) (back no))
  (plugging (front no) (back no)) (filling no) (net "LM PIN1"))
 (segment (start 103.775 59.2922) (end 104.6375 60.1547) (width 0.2) (layer "B.Cu") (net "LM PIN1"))
 (segment (start 101.806 55.0314) (end 100.6445 53.8699) (width 0.2) (layer "B.Cu") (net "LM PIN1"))
 (segment (start 103.1947 47.095) (end 103.575 47.095) (width 0.2) (layer "B.Cu") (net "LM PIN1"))
 (segment (start 102.0632 55.0314) (end 101.806 55.0314) (width 0.2) (layer "B.Cu") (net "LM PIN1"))
 (segment (start 100.6445 49.6452) (end 103.1947 47.095) (width 0.2) (layer "B.Cu") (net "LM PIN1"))
 (segment (start 103.775 58.705) (end 103.775 59.2922) (width 0.2) (layer "B.Cu") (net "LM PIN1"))
 (segment (start 100.6445 53.8699) (end 100.6445 49.6452) (width 0.2) (layer "B.Cu") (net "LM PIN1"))
 (segment (start 101.26 62.7) (end 101.26 53.5165) (width 0.2) (layer "F.Cu") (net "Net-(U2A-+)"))
 (via (at 101.26 53.5165) (size 0.6) (drill 0.3) (layers "F.Cu" "B.Cu") (capping no) (covering (front no) (back no))
  (plugging (front no) (back no)) (filling no) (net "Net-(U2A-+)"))
 (segment (start 103.575 49.635) (end 103.175 49.635) (width 0.2) (layer "B.Cu") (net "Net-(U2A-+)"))
 (segment (start 103.175 49.635) (end 101.26 51.55) (width 0.2) (layer "B.Cu") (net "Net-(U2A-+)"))
 (segment (start 101.26 51.55) (end 101.26 53.5165) (width 0.2) (layer "B.Cu") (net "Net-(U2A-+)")))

